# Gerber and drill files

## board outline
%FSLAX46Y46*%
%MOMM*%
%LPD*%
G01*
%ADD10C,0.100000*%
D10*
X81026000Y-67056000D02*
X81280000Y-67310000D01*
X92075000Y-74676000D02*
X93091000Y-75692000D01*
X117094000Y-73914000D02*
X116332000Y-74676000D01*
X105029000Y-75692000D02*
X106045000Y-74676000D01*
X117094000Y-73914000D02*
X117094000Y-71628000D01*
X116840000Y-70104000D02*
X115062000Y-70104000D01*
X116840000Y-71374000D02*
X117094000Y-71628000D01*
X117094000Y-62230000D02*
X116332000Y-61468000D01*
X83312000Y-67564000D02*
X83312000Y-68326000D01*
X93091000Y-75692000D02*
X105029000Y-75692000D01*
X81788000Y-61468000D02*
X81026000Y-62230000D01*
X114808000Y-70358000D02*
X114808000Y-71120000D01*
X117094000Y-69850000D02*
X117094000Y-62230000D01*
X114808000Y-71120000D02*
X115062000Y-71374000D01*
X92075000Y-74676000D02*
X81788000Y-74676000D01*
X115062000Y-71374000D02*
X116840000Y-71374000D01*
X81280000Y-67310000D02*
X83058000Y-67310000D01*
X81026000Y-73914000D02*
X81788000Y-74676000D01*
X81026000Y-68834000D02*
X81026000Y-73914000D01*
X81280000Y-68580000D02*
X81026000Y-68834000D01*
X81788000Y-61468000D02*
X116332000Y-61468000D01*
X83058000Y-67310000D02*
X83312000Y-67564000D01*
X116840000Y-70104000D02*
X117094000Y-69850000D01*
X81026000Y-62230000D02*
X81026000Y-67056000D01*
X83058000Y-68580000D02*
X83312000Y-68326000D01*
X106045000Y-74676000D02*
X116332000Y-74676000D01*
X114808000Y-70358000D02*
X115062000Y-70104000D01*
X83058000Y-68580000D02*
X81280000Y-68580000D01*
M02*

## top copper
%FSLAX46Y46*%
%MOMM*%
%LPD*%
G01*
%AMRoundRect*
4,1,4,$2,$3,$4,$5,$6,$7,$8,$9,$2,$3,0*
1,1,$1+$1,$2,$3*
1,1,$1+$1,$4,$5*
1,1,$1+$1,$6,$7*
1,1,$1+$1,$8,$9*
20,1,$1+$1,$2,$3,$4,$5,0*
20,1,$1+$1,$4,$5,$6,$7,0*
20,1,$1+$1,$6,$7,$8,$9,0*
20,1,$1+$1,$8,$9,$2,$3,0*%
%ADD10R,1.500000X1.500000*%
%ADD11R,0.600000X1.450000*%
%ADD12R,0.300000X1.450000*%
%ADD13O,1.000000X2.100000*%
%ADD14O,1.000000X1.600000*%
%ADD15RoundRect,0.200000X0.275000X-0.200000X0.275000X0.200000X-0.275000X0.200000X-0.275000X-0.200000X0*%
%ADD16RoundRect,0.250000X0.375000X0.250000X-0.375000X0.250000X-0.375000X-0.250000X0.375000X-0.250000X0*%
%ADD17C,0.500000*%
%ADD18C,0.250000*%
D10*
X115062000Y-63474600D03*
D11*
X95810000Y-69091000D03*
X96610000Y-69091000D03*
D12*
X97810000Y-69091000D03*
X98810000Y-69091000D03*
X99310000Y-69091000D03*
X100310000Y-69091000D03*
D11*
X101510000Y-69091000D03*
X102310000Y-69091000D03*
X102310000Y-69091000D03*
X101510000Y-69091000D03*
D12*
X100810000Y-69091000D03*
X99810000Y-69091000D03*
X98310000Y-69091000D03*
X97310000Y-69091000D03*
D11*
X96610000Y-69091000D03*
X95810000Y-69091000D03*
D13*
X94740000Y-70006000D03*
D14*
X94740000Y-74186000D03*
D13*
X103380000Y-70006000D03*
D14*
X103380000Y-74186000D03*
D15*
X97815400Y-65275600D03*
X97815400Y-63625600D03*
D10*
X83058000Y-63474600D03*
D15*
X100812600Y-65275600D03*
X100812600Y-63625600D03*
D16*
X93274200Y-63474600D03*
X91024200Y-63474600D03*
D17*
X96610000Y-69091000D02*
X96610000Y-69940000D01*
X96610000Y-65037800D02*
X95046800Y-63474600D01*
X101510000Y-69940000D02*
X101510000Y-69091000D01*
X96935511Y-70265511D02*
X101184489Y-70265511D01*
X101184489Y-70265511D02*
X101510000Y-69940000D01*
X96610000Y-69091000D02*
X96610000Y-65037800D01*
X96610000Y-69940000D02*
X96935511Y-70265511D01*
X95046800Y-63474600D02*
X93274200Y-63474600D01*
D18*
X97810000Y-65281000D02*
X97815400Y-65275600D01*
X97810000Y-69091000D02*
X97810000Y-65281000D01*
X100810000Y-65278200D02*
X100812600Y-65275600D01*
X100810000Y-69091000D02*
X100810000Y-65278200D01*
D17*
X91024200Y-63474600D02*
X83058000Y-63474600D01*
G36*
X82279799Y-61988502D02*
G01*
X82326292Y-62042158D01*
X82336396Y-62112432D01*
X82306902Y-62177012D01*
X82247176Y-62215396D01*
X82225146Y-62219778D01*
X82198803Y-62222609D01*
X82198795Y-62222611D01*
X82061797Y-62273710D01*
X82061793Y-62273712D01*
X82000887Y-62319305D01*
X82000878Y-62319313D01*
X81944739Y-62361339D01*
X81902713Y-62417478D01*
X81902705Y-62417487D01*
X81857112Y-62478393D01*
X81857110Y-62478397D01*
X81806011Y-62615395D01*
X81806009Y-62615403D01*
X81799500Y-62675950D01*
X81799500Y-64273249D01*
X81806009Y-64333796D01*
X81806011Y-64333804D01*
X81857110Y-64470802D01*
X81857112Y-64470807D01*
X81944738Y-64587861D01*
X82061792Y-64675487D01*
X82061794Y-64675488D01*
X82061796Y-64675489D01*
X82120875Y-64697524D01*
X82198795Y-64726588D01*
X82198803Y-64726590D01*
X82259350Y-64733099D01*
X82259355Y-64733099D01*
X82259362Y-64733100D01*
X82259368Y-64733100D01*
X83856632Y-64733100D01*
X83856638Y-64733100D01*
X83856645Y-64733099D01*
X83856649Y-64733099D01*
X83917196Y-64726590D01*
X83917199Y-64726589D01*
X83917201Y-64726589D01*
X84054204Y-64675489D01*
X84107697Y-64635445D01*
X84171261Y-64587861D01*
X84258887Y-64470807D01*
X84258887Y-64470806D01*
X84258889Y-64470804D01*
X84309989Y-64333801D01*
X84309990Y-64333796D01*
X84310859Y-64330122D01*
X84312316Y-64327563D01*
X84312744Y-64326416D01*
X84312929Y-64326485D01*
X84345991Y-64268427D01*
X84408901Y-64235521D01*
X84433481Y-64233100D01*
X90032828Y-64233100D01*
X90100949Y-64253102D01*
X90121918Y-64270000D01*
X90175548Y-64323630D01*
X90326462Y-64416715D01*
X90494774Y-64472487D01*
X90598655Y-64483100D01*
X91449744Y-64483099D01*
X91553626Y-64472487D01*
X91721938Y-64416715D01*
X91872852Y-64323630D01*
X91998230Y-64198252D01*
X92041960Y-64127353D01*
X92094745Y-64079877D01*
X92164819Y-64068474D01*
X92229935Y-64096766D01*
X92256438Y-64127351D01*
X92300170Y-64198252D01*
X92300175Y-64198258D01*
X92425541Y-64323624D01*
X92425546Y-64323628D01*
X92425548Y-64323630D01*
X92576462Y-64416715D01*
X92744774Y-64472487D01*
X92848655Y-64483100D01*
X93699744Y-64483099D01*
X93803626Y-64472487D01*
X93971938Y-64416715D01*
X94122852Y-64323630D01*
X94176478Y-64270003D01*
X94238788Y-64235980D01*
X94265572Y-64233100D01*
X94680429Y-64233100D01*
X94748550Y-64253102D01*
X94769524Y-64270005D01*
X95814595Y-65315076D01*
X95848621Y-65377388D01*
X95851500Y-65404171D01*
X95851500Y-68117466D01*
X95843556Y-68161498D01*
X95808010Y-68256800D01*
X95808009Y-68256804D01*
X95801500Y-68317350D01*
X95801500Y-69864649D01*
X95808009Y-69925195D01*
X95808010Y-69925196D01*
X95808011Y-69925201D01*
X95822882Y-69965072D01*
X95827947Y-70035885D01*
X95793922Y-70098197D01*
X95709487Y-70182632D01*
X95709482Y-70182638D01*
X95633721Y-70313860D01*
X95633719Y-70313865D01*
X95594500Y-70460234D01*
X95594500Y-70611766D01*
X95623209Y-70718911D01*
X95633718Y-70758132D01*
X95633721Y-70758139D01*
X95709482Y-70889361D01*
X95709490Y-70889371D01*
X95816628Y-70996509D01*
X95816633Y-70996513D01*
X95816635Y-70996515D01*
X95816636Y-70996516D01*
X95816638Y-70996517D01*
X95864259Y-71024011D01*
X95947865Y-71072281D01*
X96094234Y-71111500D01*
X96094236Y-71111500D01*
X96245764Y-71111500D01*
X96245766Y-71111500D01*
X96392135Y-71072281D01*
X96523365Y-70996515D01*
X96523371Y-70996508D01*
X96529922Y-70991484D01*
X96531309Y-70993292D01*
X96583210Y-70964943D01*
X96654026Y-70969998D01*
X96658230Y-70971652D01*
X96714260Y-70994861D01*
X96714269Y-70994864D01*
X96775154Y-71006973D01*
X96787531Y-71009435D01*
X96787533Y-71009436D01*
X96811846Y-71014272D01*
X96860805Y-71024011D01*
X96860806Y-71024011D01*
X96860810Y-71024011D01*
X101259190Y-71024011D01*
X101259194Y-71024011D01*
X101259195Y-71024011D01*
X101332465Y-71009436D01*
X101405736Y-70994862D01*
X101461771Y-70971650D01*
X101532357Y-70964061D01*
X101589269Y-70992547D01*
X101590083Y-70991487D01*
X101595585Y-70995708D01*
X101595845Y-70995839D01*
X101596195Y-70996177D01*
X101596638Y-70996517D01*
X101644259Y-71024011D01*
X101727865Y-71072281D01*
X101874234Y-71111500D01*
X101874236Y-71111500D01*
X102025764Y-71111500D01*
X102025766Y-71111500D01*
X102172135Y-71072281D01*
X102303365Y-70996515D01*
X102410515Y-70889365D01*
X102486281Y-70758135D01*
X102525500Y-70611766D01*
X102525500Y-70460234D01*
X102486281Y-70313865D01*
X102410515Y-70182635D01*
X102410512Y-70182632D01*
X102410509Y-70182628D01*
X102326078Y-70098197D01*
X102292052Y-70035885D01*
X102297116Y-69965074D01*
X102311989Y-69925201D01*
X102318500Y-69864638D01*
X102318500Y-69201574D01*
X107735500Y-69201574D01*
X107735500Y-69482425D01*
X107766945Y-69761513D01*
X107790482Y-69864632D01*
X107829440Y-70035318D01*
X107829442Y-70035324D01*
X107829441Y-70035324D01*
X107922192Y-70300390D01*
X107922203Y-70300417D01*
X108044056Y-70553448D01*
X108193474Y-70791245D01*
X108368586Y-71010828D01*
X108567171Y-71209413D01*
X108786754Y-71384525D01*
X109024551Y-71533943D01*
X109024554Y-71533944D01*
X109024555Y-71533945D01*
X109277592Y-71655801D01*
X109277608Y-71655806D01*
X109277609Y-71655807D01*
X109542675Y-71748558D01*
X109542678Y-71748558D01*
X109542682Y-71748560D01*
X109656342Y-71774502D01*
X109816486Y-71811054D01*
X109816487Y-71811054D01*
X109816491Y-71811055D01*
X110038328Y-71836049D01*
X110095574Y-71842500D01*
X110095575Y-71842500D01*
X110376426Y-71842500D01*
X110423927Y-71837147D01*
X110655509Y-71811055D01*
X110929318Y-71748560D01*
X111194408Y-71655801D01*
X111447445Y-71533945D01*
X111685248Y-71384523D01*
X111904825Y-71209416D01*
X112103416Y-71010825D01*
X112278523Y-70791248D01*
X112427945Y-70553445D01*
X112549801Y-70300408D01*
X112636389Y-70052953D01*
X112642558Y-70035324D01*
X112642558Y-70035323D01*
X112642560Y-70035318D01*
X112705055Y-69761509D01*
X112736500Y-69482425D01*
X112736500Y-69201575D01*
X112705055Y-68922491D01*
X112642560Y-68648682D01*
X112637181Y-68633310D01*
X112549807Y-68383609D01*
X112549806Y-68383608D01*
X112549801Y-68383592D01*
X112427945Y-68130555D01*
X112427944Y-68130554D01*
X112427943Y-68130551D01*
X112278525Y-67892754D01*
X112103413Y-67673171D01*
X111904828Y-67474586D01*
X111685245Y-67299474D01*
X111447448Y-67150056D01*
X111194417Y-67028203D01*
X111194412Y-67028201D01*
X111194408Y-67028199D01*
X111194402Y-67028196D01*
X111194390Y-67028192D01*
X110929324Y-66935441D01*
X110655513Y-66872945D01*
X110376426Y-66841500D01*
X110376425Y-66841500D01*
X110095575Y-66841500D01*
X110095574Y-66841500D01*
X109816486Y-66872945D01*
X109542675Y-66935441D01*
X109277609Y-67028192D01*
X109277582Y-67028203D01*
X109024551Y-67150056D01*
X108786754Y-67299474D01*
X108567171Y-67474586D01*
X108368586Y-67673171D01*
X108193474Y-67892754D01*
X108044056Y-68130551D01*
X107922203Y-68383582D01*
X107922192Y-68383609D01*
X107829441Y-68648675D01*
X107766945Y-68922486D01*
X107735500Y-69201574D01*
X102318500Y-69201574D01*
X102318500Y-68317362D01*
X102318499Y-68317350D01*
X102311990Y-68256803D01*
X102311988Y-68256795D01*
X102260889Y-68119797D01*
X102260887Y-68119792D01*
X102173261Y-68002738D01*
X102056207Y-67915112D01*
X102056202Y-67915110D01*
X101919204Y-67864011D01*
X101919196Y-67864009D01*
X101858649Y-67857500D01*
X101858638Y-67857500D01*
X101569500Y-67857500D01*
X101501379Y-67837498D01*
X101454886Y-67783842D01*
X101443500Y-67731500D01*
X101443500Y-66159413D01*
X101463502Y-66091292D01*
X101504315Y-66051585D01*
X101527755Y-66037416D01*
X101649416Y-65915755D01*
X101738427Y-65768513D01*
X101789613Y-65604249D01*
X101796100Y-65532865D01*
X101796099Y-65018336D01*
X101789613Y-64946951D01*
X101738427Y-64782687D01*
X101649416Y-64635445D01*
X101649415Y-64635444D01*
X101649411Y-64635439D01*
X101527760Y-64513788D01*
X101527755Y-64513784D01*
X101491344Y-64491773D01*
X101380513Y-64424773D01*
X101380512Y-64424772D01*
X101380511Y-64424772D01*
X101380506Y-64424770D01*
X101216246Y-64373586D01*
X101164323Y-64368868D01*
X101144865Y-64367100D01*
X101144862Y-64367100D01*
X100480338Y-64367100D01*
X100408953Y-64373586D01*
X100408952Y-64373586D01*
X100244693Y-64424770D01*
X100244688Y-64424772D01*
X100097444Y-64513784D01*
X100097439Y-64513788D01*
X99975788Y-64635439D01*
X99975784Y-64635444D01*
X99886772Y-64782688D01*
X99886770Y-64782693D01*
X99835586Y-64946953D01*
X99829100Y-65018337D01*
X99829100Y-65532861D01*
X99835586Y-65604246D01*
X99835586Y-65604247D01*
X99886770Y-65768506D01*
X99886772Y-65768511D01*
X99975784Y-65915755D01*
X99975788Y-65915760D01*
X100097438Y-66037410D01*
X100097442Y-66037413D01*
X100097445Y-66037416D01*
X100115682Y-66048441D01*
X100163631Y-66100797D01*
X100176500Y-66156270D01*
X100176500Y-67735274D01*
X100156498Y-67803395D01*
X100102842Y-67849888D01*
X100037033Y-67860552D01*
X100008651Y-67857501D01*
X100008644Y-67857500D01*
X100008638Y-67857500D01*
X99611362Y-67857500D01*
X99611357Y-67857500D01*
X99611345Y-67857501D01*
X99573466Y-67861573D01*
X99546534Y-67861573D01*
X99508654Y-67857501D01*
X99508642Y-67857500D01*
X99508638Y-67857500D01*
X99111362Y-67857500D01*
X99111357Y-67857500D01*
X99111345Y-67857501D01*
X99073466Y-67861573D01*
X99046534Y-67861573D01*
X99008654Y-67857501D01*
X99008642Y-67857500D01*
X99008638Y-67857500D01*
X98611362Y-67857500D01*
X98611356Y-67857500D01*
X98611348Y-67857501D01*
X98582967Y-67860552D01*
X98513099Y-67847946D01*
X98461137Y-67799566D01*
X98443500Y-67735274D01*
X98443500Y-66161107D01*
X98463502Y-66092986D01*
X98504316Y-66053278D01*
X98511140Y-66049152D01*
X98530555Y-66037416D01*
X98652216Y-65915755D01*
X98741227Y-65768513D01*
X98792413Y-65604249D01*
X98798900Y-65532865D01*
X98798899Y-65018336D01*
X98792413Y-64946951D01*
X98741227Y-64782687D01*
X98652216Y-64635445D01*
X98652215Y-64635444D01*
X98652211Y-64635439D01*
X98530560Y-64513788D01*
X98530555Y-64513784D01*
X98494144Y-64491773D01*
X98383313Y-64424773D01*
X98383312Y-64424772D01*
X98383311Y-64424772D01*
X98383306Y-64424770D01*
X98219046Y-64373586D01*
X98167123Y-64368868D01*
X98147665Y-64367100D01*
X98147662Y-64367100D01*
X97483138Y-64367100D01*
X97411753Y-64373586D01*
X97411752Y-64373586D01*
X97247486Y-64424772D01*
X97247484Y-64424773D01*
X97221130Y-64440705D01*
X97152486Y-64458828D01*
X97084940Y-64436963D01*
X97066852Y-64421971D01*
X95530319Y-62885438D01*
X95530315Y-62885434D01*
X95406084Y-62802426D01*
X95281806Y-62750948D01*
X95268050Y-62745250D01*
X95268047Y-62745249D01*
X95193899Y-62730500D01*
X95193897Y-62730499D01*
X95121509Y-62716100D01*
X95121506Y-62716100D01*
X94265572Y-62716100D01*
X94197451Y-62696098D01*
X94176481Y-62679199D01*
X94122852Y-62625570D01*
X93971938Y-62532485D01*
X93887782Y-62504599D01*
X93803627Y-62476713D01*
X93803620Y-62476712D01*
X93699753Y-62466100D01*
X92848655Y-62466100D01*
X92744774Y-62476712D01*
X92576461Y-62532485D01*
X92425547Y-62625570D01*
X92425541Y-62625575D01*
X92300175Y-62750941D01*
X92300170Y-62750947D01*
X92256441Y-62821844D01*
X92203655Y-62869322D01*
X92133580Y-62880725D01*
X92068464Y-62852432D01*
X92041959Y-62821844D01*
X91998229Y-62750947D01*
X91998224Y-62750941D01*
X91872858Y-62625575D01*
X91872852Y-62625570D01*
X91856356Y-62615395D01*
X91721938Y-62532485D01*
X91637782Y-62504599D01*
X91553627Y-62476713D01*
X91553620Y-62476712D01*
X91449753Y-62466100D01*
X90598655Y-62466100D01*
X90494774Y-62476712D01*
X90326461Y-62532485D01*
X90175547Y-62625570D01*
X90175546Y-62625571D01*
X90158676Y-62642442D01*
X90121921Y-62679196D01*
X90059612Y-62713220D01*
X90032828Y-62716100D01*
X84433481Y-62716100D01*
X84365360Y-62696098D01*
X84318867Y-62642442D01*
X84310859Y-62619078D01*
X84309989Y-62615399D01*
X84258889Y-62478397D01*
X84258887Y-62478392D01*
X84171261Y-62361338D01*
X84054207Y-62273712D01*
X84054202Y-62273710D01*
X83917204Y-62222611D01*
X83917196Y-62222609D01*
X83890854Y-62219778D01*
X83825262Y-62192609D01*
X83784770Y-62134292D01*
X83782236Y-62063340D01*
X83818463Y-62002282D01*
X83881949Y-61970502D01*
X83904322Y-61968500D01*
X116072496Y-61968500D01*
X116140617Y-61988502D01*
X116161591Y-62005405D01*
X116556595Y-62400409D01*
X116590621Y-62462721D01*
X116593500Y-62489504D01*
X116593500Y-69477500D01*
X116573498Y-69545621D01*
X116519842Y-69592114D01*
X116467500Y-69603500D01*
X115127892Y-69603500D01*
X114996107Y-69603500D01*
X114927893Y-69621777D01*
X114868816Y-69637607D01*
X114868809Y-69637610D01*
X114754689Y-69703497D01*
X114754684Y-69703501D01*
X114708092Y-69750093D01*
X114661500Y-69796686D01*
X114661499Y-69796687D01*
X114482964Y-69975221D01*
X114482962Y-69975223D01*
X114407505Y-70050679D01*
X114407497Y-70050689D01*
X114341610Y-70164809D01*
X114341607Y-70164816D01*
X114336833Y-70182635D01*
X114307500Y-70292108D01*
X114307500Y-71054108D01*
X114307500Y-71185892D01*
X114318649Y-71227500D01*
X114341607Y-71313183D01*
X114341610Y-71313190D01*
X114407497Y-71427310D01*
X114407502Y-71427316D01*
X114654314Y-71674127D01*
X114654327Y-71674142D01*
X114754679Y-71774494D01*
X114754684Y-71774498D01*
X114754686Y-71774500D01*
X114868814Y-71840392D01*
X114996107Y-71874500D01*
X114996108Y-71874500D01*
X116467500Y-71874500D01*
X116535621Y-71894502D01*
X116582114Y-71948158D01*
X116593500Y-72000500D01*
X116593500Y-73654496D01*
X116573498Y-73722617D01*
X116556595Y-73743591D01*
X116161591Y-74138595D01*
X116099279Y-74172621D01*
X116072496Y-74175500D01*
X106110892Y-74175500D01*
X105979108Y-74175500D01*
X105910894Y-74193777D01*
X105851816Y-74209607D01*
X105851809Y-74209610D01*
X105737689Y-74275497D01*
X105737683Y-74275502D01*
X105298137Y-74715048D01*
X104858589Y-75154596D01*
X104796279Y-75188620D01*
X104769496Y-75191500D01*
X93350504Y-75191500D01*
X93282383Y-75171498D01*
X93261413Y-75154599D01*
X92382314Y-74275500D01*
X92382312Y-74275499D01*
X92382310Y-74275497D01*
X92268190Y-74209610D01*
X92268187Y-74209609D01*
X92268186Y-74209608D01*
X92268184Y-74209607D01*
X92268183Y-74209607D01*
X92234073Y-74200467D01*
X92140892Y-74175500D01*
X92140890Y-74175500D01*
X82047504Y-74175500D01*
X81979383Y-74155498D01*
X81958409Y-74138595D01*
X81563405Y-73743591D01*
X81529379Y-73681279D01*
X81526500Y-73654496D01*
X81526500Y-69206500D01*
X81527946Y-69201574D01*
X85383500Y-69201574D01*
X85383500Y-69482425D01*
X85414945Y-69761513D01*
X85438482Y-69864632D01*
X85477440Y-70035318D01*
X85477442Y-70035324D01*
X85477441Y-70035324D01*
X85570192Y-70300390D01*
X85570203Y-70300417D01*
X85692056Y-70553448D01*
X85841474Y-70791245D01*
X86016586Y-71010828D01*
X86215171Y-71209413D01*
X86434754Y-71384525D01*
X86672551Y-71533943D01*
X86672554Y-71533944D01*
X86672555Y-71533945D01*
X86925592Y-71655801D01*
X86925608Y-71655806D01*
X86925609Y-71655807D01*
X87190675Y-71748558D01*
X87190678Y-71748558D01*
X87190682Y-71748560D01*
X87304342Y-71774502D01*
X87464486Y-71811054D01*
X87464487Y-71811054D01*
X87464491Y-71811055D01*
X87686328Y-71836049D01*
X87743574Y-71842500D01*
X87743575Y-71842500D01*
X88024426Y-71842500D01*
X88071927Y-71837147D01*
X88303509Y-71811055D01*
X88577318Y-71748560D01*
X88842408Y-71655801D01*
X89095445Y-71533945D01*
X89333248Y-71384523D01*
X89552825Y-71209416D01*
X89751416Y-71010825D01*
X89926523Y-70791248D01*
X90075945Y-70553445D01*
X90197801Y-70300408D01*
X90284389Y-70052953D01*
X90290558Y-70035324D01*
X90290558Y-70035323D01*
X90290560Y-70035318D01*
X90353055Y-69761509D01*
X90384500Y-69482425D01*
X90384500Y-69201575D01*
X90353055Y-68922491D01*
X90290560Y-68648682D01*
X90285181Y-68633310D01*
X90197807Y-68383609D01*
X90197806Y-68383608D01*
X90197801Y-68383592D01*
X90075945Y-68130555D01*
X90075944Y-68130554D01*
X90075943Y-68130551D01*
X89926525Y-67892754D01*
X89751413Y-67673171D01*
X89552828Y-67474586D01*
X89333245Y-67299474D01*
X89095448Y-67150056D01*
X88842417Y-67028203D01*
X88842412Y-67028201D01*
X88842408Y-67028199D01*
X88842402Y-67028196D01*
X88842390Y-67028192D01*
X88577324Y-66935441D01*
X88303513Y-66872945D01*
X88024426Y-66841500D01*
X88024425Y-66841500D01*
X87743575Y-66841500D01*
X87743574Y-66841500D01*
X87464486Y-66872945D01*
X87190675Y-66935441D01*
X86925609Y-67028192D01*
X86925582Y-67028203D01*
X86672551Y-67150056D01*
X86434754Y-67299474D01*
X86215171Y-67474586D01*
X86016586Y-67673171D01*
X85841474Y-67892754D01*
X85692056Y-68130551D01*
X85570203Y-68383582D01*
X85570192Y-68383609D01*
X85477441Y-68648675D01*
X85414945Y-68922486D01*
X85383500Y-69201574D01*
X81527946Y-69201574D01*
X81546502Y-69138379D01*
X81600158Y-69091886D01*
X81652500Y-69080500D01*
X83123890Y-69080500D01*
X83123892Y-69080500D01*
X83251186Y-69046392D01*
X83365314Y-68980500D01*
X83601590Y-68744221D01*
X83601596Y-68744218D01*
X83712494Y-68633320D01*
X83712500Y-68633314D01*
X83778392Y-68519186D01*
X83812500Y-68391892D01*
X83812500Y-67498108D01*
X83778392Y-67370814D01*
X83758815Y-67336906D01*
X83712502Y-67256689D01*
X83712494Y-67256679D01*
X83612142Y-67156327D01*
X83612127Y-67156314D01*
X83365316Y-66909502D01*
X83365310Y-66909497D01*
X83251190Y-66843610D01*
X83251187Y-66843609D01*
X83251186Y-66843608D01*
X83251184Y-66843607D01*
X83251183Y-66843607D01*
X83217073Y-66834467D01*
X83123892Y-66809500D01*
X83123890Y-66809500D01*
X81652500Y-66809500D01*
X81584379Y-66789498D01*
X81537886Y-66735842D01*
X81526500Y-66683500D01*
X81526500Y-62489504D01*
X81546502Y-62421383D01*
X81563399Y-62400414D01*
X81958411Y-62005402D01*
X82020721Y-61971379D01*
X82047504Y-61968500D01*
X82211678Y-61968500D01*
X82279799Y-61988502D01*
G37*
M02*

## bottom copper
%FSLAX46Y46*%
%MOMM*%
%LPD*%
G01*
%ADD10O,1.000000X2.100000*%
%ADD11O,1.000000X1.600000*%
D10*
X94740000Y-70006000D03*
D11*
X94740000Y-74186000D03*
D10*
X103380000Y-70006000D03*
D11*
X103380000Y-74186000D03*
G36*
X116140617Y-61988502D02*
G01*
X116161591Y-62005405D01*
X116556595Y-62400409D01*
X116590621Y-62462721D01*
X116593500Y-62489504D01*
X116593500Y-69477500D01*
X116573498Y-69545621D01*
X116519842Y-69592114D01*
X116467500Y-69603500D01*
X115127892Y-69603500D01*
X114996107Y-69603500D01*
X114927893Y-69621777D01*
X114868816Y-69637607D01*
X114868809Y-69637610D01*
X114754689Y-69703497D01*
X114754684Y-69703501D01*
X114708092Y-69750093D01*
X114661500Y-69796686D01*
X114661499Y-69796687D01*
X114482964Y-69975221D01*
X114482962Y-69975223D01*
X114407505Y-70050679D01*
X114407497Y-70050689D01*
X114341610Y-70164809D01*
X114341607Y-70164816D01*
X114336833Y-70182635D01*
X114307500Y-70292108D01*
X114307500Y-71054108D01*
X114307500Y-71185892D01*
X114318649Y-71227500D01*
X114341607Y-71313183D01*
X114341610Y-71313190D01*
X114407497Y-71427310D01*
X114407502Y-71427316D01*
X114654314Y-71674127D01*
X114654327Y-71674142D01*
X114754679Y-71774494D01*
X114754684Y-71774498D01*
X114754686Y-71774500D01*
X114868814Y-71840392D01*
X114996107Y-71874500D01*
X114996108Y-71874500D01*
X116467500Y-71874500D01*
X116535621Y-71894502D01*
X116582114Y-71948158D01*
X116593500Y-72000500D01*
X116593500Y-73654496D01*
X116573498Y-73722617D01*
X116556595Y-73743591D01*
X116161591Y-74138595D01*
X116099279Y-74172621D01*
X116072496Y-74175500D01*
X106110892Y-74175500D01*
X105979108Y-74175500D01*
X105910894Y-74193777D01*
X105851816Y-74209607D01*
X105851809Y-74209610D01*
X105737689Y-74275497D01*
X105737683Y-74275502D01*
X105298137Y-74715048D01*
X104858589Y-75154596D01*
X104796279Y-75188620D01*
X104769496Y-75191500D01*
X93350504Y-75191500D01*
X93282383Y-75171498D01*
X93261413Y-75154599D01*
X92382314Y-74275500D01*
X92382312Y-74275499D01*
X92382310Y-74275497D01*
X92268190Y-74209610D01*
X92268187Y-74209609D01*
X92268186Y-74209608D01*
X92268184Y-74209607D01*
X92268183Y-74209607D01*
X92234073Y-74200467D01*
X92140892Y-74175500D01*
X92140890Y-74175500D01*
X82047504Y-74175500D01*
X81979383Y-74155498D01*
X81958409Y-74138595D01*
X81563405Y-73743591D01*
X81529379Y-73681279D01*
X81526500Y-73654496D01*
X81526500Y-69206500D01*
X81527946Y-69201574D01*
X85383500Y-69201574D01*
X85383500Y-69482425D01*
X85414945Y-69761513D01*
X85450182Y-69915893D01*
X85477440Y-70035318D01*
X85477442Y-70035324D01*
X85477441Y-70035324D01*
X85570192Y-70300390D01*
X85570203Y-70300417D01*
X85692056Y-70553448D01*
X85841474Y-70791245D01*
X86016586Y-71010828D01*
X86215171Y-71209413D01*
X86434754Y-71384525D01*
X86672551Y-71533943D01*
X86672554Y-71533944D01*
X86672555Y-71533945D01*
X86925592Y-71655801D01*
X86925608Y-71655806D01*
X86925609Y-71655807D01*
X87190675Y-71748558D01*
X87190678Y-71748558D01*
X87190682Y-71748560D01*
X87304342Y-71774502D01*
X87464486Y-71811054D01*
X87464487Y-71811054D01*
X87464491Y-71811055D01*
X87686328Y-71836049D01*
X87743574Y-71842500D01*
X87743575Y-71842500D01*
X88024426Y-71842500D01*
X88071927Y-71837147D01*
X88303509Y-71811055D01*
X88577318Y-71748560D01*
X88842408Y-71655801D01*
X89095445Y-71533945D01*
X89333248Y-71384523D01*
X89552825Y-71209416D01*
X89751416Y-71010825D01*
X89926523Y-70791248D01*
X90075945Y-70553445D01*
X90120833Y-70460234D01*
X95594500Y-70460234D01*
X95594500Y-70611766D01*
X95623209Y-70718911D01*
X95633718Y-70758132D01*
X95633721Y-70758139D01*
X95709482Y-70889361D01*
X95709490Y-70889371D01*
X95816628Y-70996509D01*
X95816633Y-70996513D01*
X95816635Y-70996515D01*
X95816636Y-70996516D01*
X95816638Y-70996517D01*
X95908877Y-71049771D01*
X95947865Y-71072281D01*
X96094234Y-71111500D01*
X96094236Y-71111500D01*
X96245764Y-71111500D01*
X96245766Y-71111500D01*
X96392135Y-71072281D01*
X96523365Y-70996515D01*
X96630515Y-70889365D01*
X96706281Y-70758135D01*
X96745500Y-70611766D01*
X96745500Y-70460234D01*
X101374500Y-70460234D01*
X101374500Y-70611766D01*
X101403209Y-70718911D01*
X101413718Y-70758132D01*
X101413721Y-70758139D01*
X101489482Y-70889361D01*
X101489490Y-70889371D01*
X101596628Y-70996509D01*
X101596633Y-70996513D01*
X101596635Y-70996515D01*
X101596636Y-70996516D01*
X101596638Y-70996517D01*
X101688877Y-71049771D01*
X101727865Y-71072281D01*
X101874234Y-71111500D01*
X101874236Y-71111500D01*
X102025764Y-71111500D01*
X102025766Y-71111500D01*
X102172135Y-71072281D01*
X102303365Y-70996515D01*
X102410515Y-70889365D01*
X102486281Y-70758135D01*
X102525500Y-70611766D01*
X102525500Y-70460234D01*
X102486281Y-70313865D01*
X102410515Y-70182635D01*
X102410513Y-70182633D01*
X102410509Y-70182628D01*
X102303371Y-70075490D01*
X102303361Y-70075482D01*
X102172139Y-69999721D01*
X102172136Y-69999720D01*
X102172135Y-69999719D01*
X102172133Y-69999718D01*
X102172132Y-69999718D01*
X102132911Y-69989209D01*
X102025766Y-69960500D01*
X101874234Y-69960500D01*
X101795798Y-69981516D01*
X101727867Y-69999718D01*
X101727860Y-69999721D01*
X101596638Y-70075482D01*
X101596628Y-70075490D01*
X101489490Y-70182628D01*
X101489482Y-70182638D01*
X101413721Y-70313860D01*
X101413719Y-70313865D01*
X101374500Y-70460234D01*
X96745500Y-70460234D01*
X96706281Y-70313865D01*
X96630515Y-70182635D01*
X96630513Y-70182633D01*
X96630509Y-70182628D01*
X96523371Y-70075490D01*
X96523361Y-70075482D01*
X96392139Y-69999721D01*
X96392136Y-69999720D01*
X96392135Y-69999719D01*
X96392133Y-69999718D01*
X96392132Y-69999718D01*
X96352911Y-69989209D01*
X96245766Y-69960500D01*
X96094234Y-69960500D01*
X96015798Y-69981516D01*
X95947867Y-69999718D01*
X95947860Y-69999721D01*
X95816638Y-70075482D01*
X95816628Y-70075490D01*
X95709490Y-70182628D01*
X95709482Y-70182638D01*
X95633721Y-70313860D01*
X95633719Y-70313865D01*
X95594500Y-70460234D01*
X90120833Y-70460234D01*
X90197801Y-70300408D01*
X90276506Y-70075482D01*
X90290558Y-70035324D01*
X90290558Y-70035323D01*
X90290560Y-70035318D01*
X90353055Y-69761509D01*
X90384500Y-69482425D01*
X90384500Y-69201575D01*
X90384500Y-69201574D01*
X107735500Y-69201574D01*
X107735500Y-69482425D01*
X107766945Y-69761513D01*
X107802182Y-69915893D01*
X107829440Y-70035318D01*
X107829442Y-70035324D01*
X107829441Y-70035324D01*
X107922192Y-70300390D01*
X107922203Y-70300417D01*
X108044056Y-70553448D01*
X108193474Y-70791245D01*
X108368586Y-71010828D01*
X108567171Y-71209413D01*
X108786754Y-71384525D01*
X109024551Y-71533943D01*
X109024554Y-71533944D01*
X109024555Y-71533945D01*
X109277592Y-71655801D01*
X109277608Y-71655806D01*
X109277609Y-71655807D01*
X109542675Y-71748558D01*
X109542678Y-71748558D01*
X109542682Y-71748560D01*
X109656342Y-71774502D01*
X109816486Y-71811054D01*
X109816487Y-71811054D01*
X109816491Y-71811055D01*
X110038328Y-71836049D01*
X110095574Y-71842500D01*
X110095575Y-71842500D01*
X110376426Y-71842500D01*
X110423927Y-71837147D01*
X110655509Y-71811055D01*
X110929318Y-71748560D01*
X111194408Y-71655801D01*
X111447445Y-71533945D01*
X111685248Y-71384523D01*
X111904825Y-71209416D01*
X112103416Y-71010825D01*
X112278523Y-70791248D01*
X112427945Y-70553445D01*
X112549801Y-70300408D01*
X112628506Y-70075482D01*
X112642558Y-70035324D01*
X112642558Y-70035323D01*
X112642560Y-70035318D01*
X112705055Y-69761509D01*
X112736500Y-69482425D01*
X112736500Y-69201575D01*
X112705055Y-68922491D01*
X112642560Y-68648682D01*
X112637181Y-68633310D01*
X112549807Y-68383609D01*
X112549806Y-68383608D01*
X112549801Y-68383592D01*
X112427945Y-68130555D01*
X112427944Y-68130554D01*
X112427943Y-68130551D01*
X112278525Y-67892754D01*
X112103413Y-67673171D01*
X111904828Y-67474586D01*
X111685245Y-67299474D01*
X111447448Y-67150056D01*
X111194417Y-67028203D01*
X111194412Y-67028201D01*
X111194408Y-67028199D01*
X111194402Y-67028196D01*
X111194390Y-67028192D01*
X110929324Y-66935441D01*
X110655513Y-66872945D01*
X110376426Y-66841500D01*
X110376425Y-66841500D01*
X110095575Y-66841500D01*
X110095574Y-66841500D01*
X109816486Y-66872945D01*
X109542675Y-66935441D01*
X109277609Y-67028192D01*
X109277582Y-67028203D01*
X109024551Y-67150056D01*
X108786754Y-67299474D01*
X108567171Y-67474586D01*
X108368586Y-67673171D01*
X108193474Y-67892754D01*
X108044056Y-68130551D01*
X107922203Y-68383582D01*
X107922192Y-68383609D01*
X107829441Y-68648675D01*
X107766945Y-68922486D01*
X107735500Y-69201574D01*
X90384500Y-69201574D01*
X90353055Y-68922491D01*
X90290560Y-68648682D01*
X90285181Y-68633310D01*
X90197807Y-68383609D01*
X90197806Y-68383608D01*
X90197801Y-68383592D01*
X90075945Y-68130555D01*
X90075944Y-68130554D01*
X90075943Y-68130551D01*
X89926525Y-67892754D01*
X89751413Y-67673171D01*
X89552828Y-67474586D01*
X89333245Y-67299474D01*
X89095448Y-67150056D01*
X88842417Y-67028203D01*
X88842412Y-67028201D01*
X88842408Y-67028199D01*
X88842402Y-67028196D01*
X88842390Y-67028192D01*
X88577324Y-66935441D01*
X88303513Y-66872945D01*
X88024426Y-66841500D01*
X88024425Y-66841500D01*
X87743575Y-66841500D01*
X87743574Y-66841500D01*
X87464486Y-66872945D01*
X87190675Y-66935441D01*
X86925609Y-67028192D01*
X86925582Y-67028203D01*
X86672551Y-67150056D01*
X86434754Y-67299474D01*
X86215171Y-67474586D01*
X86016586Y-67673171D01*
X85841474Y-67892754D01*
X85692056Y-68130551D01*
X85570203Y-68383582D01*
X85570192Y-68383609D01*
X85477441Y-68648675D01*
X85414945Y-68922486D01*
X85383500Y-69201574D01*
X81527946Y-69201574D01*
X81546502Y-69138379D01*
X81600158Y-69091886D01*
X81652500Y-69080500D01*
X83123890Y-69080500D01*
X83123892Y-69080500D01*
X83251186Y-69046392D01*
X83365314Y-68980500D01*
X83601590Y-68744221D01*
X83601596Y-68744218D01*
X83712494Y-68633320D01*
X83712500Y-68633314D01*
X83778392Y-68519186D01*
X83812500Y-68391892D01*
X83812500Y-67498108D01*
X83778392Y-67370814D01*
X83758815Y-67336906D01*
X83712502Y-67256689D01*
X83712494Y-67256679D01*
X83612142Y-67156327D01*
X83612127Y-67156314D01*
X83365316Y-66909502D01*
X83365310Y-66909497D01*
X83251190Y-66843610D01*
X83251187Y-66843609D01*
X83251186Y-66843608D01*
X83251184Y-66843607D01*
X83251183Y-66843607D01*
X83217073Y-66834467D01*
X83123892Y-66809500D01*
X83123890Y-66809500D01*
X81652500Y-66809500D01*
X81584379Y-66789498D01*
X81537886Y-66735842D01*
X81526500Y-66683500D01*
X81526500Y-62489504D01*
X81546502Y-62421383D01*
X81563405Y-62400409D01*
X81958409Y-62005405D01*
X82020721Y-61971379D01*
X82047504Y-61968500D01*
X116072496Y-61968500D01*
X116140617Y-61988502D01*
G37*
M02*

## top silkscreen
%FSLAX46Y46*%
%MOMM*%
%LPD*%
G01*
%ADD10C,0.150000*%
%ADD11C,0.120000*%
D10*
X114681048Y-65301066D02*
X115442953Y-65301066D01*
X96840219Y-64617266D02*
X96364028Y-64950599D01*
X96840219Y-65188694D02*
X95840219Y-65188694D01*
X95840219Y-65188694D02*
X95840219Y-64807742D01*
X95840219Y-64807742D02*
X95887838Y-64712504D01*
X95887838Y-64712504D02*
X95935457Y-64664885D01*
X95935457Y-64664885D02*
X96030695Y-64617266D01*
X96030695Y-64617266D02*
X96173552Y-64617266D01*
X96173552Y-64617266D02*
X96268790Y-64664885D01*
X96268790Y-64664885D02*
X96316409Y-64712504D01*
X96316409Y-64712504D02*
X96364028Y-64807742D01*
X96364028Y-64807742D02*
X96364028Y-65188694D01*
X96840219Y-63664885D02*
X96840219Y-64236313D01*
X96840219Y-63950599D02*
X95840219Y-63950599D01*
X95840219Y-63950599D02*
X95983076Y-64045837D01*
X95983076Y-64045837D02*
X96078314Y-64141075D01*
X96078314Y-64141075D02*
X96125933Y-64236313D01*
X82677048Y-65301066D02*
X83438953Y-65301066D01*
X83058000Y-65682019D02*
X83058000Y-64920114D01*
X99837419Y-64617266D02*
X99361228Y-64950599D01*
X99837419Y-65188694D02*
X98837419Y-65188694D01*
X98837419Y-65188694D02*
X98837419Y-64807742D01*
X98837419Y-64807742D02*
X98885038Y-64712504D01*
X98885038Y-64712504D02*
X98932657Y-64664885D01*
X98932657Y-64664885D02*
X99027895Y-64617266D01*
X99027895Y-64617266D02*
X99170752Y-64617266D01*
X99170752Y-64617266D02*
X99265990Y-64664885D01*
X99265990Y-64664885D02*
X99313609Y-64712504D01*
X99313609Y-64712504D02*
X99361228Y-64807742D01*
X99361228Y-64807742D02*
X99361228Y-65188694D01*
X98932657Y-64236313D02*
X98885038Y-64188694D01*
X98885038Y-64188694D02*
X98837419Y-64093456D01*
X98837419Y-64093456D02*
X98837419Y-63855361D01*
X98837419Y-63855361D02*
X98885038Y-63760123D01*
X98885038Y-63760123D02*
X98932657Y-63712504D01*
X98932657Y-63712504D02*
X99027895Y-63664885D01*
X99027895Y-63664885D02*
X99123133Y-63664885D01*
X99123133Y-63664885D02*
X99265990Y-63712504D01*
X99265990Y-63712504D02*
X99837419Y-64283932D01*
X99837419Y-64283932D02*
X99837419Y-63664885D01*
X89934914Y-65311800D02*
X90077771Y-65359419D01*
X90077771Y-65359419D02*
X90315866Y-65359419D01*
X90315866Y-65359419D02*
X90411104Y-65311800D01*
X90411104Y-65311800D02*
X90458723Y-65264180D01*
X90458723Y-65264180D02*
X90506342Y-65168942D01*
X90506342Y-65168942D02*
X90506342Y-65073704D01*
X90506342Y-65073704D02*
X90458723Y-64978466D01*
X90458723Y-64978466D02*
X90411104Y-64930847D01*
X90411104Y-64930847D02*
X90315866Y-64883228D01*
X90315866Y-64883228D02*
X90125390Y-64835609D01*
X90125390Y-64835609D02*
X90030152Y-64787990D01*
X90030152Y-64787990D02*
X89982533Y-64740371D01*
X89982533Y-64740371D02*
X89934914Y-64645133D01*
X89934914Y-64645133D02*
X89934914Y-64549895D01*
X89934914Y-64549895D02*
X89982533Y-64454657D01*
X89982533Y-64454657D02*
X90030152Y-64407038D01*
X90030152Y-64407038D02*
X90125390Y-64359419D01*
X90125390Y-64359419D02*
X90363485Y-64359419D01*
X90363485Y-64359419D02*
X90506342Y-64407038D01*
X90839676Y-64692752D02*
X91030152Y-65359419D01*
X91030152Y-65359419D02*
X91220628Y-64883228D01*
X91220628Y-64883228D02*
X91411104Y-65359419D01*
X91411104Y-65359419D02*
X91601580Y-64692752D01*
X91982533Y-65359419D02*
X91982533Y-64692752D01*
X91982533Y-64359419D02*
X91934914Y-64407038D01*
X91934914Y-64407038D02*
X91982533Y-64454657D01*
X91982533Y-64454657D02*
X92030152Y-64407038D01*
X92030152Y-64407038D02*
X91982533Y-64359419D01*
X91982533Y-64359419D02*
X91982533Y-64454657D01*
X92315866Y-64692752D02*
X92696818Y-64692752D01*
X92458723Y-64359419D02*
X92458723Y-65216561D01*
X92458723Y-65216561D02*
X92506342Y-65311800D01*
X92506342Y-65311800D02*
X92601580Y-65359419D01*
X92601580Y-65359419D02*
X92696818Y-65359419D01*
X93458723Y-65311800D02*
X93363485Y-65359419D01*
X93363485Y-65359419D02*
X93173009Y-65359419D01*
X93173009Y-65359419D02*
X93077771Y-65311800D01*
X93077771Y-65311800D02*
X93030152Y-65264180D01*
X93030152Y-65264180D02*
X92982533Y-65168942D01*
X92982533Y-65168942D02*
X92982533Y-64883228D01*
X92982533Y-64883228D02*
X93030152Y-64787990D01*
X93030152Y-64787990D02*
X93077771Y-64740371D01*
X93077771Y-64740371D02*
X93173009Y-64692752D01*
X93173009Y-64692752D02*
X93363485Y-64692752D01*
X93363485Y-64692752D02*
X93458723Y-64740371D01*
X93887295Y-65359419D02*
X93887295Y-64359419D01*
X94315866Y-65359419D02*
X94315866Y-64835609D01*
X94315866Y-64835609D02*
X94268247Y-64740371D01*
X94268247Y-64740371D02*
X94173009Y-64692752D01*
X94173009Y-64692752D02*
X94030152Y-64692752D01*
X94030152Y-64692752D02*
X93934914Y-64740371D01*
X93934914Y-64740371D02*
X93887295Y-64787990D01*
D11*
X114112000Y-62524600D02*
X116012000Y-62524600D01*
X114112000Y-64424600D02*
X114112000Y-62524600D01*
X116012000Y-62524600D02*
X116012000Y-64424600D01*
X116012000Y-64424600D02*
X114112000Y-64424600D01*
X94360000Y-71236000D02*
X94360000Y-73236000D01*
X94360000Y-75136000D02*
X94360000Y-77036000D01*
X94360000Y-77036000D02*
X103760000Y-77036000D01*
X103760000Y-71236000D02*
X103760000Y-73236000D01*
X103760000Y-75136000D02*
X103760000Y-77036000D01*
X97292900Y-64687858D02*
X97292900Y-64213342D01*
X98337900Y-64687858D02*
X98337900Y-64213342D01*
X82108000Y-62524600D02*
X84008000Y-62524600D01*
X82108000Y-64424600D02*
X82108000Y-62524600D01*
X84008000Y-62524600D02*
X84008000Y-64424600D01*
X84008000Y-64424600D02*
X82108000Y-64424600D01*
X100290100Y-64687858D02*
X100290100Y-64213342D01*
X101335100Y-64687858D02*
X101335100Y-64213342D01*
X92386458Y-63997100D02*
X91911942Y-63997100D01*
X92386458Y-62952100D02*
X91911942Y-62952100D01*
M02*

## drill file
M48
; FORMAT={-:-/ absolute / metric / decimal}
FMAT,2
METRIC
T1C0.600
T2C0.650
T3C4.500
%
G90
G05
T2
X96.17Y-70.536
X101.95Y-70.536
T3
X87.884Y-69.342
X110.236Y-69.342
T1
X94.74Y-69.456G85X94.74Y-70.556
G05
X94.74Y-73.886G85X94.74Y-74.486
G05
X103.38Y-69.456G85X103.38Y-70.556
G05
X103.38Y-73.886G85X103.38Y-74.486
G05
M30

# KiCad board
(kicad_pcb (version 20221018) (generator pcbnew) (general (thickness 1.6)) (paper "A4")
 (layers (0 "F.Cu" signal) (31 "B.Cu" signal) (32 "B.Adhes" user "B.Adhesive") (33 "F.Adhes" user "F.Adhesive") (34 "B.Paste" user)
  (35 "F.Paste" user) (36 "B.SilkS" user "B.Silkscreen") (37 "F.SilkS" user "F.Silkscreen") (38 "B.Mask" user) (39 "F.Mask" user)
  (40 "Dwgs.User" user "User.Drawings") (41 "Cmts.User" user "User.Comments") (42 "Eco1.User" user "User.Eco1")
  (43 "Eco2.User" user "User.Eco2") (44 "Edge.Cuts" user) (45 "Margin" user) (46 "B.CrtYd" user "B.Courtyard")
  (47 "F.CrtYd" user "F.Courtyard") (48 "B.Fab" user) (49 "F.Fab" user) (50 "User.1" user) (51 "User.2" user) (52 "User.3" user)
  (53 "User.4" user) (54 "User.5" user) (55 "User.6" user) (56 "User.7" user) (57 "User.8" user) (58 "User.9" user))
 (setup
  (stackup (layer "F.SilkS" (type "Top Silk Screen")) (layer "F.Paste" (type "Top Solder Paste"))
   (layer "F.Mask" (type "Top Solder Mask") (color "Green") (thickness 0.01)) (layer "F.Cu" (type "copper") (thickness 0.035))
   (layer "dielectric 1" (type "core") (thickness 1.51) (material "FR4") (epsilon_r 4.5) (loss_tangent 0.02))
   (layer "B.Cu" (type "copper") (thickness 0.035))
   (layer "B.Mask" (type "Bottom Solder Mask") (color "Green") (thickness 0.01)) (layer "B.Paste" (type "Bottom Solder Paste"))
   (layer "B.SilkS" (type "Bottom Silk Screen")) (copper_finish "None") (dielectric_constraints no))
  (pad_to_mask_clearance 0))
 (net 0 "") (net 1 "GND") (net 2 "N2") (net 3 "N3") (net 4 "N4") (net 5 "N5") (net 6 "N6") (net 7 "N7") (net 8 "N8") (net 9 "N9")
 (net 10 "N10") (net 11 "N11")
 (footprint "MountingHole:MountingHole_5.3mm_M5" (layer "F.Cu") (at 87.884 69.342)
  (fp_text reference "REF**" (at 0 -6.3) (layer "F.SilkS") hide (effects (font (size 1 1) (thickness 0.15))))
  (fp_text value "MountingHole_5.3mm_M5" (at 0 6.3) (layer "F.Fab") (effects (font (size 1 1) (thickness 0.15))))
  (pad "" np_thru_hole circle (at 0 0) (size 4.5 4.5) (drill 4.5) (layers "F&B.Cu" "*.Mask")))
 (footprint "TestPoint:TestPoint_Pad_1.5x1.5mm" (layer "F.Cu") (at 115.062 63.4746)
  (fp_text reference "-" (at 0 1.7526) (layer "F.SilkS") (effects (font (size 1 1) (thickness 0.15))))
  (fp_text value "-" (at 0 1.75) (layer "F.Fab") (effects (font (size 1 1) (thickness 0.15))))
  (fp_line (start -0.95 -0.95) (end 0.95 -0.95) (stroke (width 0.12) (type solid)) (layer "F.SilkS"))
  (fp_line (start -0.95 0.95) (end -0.95 -0.95) (stroke (width 0.12) (type solid)) (layer "F.SilkS"))
  (fp_line (start 0.95 -0.95) (end 0.95 0.95) (stroke (width 0.12) (type solid)) (layer "F.SilkS"))
  (fp_line (start 0.95 0.95) (end -0.95 0.95) (stroke (width 0.12) (type solid)) (layer "F.SilkS"))
  (pad "1" smd rect (at 0 0) (size 1.5 1.5) (layers "F.Cu" "F.Mask") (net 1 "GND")))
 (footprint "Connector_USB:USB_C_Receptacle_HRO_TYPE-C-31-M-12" (layer "F.Cu") (at 99.06 73.136)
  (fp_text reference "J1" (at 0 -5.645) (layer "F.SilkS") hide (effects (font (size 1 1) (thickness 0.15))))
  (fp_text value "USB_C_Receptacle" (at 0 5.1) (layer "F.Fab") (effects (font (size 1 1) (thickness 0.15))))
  (fp_line (start -4.7 -1.9) (end -4.7 0.1) (stroke (width 0.12) (type solid)) (layer "F.SilkS"))
  (fp_line (start -4.7 2) (end -4.7 3.9) (stroke (width 0.12) (type solid)) (layer "F.SilkS"))
  (fp_line (start -4.7 3.9) (end 4.7 3.9) (stroke (width 0.12) (type solid)) (layer "F.SilkS"))
  (fp_line (start 4.7 -1.9) (end 4.7 0.1) (stroke (width 0.12) (type solid)) (layer "F.SilkS"))
  (fp_line (start 4.7 2) (end 4.7 3.9) (stroke (width 0.12) (type solid)) (layer "F.SilkS"))
  (pad "" np_thru_hole circle (at -2.89 -2.6) (size 0.65 0.65) (drill 0.65) (layers "*.Cu" "*.Mask"))
  (pad "" np_thru_hole circle (at 2.89 -2.6) (size 0.65 0.65) (drill 0.65) (layers "*.Cu" "*.Mask"))
  (pad "A1" smd rect (at -3.25 -4.045) (size 0.6 1.45) (layers "F.Cu" "F.Paste" "F.Mask") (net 1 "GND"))
  (pad "A4" smd rect (at -2.45 -4.045) (size 0.6 1.45) (layers "F.Cu" "F.Paste" "F.Mask") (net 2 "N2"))
  (pad "A5" smd rect (at -1.25 -4.045) (size 0.3 1.45) (layers "F.Cu" "F.Paste" "F.Mask") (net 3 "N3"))
  (pad "A6" smd rect (at -0.25 -4.045) (size 0.3 1.45) (layers "F.Cu" "F.Paste" "F.Mask") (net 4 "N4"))
  (pad "A7" smd rect (at 0.25 -4.045) (size 0.3 1.45) (layers "F.Cu" "F.Paste" "F.Mask") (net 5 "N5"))
  (pad "A8" smd rect (at 1.25 -4.045) (size 0.3 1.45) (layers "F.Cu" "F.Paste" "F.Mask") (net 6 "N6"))
  (pad "A9" smd rect (at 2.45 -4.045) (size 0.6 1.45) (layers "F.Cu" "F.Paste" "F.Mask") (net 2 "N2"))
  (pad "A12" smd rect (at 3.25 -4.045) (size 0.6 1.45) (layers "F.Cu" "F.Paste" "F.Mask") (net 1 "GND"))
  (pad "B1" smd rect (at 3.25 -4.045) (size 0.6 1.45) (layers "F.Cu" "F.Paste" "F.Mask") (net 1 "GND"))
  (pad "B4" smd rect (at 2.45 -4.045) (size 0.6 1.45) (layers "F.Cu" "F.Paste" "F.Mask") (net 2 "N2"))
  (pad "B5" smd rect (at 1.75 -4.045) (size 0.3 1.45) (layers "F.Cu" "F.Paste" "F.Mask") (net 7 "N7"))
  (pad "B6" smd rect (at 0.75 -4.045) (size 0.3 1.45) (layers "F.Cu" "F.Paste" "F.Mask") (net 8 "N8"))
  (pad "B7" smd rect (at -0.75 -4.045) (size 0.3 1.45) (layers "F.Cu" "F.Paste" "F.Mask") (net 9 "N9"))
  (pad "B8" smd rect (at -1.75 -4.045) (size 0.3 1.45) (layers "F.Cu" "F.Paste" "F.Mask") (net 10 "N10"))
  (pad "B9" smd rect (at -2.45 -4.045) (size 0.6 1.45) (layers "F.Cu" "F.Paste" "F.Mask") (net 2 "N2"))
  (pad "B12" smd rect (at -3.25 -4.045) (size 0.6 1.45) (layers "F.Cu" "F.Paste" "F.Mask") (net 1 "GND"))
  (pad "S1" thru_hole oval (at -4.32 -3.13) (size 1 2.1) (drill oval 0.6 1.7) (layers "*.Cu" "*.Mask") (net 1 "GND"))
  (pad "S1" thru_hole oval (at -4.32 1.05) (size 1 1.6) (drill oval 0.6 1.2) (layers "*.Cu" "*.Mask") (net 1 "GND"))
  (pad "S1" thru_hole oval (at 4.32 -3.13) (size 1 2.1) (drill oval 0.6 1.7) (layers "*.Cu" "*.Mask") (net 1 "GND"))
  (pad "S1" thru_hole oval (at 4.32 1.05) (size 1 1.6) (drill oval 0.6 1.2) (layers "*.Cu" "*.Mask") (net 1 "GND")))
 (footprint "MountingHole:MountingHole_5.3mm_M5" (layer "F.Cu") (at 110.236 69.342)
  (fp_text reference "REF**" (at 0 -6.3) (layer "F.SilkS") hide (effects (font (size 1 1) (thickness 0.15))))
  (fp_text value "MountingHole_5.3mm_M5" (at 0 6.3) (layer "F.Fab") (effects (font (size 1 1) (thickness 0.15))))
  (pad "" np_thru_hole circle (at 0 0) (size 4.5 4.5) (drill 4.5) (layers "F&B.Cu" "*.Mask")))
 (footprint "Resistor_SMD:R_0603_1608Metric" (layer "F.Cu") (at 97.8154 64.4506 90)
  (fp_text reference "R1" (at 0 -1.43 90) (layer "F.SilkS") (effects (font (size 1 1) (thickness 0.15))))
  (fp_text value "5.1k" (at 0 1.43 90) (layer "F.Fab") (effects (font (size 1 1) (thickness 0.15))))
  (fp_line (start -0.237258 -0.5225) (end 0.237258 -0.5225) (stroke (width 0.12) (type solid)) (layer "F.SilkS"))
  (fp_line (start -0.237258 0.5225) (end 0.237258 0.5225) (stroke (width 0.12) (type solid)) (layer "F.SilkS"))
  (pad "1" smd roundrect (at -0.825 0 90) (size 0.8 0.95) (layers "F.Cu" "F.Paste" "F.Mask") (roundrect_rratio 0.25) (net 3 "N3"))
  (pad "2" smd roundrect (at 0.825 0 90) (size 0.8 0.95) (layers "F.Cu" "F.Paste" "F.Mask") (roundrect_rratio 0.25) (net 1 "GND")))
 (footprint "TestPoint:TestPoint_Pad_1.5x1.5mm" (layer "F.Cu") (at 83.058 63.4746)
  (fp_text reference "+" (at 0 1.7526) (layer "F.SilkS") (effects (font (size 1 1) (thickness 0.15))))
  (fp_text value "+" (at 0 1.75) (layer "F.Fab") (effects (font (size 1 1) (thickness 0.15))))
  (fp_line (start -0.95 -0.95) (end 0.95 -0.95) (stroke (width 0.12) (type solid)) (layer "F.SilkS"))
  (fp_line (start -0.95 0.95) (end -0.95 -0.95) (stroke (width 0.12) (type solid)) (layer "F.SilkS"))
  (fp_line (start 0.95 -0.95) (end 0.95 0.95) (stroke (width 0.12) (type solid)) (layer "F.SilkS"))
  (fp_line (start 0.95 0.95) (end -0.95 0.95) (stroke (width 0.12) (type solid)) (layer "F.SilkS"))
  (pad "1" smd rect (at 0 0) (size 1.5 1.5) (layers "F.Cu" "F.Mask") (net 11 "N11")))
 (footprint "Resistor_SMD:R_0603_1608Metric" (layer "F.Cu") (at 100.8126 64.4506 90)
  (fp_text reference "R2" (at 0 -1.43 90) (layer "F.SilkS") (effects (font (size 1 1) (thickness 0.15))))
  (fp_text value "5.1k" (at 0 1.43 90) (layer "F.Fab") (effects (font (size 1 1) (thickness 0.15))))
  (fp_line (start -0.237258 -0.5225) (end 0.237258 -0.5225) (stroke (width 0.12) (type solid)) (layer "F.SilkS"))
  (fp_line (start -0.237258 0.5225) (end 0.237258 0.5225) (stroke (width 0.12) (type solid)) (layer "F.SilkS"))
  (pad "1" smd roundrect (at -0.825 0 90) (size 0.8 0.95) (layers "F.Cu" "F.Paste" "F.Mask") (roundrect_rratio 0.25) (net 7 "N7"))
  (pad "2" smd roundrect (at 0.825 0 90) (size 0.8 0.95) (layers "F.Cu" "F.Paste" "F.Mask") (roundrect_rratio 0.25) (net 1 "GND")))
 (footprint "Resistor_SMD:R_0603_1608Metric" (layer "F.Cu") (at 92.1492 63.4746 180)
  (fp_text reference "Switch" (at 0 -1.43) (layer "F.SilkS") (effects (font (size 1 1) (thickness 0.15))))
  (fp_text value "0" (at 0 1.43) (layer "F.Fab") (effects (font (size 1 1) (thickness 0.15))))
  (fp_line (start -0.237258 -0.5225) (end 0.237258 -0.5225) (stroke (width 0.12) (type solid)) (layer "F.SilkS"))
  (fp_line (start -0.237258 0.5225) (end 0.237258 0.5225) (stroke (width 0.12) (type solid)) (layer "F.SilkS"))
  (pad "1" smd roundrect (at -1.125 0 180) (size 1.25 1) (layers "F.Cu" "F.Paste" "F.Mask") (roundrect_rratio 0.25) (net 2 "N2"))
  (pad "2" smd roundrect (at 1.125 0 180) (size 1.25 1) (layers "F.Cu" "F.Paste" "F.Mask") (roundrect_rratio 0.25) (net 11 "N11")))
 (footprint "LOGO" (layer "B.Cu") (at 111.0488 63.4492 180)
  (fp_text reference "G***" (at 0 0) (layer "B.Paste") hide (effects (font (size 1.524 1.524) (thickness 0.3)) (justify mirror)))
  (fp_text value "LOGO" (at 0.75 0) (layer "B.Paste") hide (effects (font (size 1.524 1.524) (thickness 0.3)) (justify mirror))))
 (gr_line (start 81.026 67.056) (end 81.28 67.31) (stroke (width 0.1) (type solid)) (layer "Edge.Cuts"))
 (gr_line (start 92.075 74.676) (end 93.091 75.692) (stroke (width 0.1) (type solid)) (layer "Edge.Cuts"))
 (gr_line (start 117.094 73.914) (end 116.332 74.676) (stroke (width 0.1) (type solid)) (layer "Edge.Cuts"))
 (gr_line (start 105.029 75.692) (end 106.045 74.676) (stroke (width 0.1) (type solid)) (layer "Edge.Cuts"))
 (gr_line (start 117.094 73.914) (end 117.094 71.628) (stroke (width 0.1) (type solid)) (layer "Edge.Cuts"))
 (gr_line (start 116.84 70.104) (end 115.062 70.104) (stroke (width 0.1) (type solid)) (layer "Edge.Cuts"))
 (gr_line (start 116.84 71.374) (end 117.094 71.628) (stroke (width 0.1) (type solid)) (layer "Edge.Cuts"))
 (gr_line (start 117.094 62.23) (end 116.332 61.468) (stroke (width 0.1) (type solid)) (layer "Edge.Cuts"))
 (gr_line (start 83.312 67.564) (end 83.312 68.326) (stroke (width 0.1) (type solid)) (layer "Edge.Cuts"))
 (gr_line (start 93.091 75.692) (end 105.029 75.692) (stroke (width 0.1) (type solid)) (layer "Edge.Cuts"))
 (gr_line (start 81.788 61.468) (end 81.026 62.23) (stroke (width 0.1) (type solid)) (layer "Edge.Cuts"))
 (gr_line (start 114.808 70.358) (end 114.808 71.12) (stroke (width 0.1) (type solid)) (layer "Edge.Cuts"))
 (gr_line (start 117.094 69.85) (end 117.094 62.23) (stroke (width 0.1) (type solid)) (layer "Edge.Cuts"))
 (gr_line (start 114.808 71.12) (end 115.062 71.374) (stroke (width 0.1) (type solid)) (layer "Edge.Cuts"))
 (gr_line (start 92.075 74.676) (end 81.788 74.676) (stroke (width 0.1) (type solid)) (layer "Edge.Cuts"))
 (gr_line (start 115.062 71.374) (end 116.84 71.374) (stroke (width 0.1) (type solid)) (layer "Edge.Cuts"))
 (gr_line (start 81.28 67.31) (end 83.058 67.31) (stroke (width 0.1) (type solid)) (layer "Edge.Cuts"))
 (gr_line (start 81.026 73.914) (end 81.788 74.676) (stroke (width 0.1) (type solid)) (layer "Edge.Cuts"))
 (gr_line (start 81.026 68.834) (end 81.026 73.914) (stroke (width 0.1) (type solid)) (layer "Edge.Cuts"))
 (gr_line (start 81.28 68.58) (end 81.026 68.834) (stroke (width 0.1) (type solid)) (layer "Edge.Cuts"))
 (gr_line (start 81.788 61.468) (end 116.332 61.468) (stroke (width 0.1) (type solid)) (layer "Edge.Cuts"))
 (gr_line (start 83.058 67.31) (end 83.312 67.564) (stroke (width 0.1) (type solid)) (layer "Edge.Cuts"))
 (gr_line (start 116.84 70.104) (end 117.094 69.85) (stroke (width 0.1) (type solid)) (layer "Edge.Cuts"))
 (gr_line (start 81.026 62.23) (end 81.026 67.056) (stroke (width 0.1) (type solid)) (layer "Edge.Cuts"))
 (gr_line (start 83.058 68.58) (end 83.312 68.326) (stroke (width 0.1) (type solid)) (layer "Edge.Cuts"))
 (gr_line (start 106.045 74.676) (end 116.332 74.676) (stroke (width 0.1) (type solid)) (layer "Edge.Cuts"))
 (gr_line (start 114.808 70.358) (end 115.062 70.104) (stroke (width 0.1) (type solid)) (layer "Edge.Cuts"))
 (gr_line (start 83.058 68.58) (end 81.28 68.58) (stroke (width 0.1) (type solid)) (layer "Edge.Cuts"))
 (segment (start 96.61 69.091) (end 96.61 69.94) (width 0.5) (layer "F.Cu") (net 2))
 (segment (start 96.61 65.0378) (end 95.0468 63.4746) (width 0.5) (layer "F.Cu") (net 2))
 (segment (start 101.51 69.94) (end 101.51 69.091) (width 0.5) (layer "F.Cu") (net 2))
 (segment (start 96.935511 70.265511) (end 101.184489 70.265511) (width 0.5) (layer "F.Cu") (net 2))
 (segment (start 101.184489 70.265511) (end 101.51 69.94) (width 0.5) (layer "F.Cu") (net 2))
 (segment (start 96.61 69.091) (end 96.61 65.0378) (width 0.5) (layer "F.Cu") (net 2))
 (segment (start 96.61 69.94) (end 96.935511 70.265511) (width 0.5) (layer "F.Cu") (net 2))
 (segment (start 95.0468 63.4746) (end 93.2742 63.4746) (width 0.5) (layer "F.Cu") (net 2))
 (segment (start 97.81 65.281) (end 97.8154 65.2756) (width 0.25) (layer "F.Cu") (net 3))
 (segment (start 97.81 69.091) (end 97.81 65.281) (width 0.25) (layer "F.Cu") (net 3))
 (segment (start 100.81 65.2782) (end 100.8126 65.2756) (width 0.25) (layer "F.Cu") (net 7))
 (segment (start 100.81 69.091) (end 100.81 65.2782) (width 0.25) (layer "F.Cu") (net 7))
 (segment (start 91.0242 63.4746) (end 83.058 63.4746) (width 0.5) (layer "F.Cu") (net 11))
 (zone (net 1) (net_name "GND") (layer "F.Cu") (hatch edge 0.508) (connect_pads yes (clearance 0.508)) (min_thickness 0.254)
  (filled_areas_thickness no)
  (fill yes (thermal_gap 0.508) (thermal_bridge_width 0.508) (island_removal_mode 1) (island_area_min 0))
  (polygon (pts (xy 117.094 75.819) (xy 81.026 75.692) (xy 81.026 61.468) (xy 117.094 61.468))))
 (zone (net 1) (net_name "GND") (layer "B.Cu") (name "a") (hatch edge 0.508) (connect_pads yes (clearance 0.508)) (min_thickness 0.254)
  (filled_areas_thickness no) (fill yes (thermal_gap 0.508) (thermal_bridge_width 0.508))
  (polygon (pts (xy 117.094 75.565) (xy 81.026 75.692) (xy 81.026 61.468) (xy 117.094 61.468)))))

